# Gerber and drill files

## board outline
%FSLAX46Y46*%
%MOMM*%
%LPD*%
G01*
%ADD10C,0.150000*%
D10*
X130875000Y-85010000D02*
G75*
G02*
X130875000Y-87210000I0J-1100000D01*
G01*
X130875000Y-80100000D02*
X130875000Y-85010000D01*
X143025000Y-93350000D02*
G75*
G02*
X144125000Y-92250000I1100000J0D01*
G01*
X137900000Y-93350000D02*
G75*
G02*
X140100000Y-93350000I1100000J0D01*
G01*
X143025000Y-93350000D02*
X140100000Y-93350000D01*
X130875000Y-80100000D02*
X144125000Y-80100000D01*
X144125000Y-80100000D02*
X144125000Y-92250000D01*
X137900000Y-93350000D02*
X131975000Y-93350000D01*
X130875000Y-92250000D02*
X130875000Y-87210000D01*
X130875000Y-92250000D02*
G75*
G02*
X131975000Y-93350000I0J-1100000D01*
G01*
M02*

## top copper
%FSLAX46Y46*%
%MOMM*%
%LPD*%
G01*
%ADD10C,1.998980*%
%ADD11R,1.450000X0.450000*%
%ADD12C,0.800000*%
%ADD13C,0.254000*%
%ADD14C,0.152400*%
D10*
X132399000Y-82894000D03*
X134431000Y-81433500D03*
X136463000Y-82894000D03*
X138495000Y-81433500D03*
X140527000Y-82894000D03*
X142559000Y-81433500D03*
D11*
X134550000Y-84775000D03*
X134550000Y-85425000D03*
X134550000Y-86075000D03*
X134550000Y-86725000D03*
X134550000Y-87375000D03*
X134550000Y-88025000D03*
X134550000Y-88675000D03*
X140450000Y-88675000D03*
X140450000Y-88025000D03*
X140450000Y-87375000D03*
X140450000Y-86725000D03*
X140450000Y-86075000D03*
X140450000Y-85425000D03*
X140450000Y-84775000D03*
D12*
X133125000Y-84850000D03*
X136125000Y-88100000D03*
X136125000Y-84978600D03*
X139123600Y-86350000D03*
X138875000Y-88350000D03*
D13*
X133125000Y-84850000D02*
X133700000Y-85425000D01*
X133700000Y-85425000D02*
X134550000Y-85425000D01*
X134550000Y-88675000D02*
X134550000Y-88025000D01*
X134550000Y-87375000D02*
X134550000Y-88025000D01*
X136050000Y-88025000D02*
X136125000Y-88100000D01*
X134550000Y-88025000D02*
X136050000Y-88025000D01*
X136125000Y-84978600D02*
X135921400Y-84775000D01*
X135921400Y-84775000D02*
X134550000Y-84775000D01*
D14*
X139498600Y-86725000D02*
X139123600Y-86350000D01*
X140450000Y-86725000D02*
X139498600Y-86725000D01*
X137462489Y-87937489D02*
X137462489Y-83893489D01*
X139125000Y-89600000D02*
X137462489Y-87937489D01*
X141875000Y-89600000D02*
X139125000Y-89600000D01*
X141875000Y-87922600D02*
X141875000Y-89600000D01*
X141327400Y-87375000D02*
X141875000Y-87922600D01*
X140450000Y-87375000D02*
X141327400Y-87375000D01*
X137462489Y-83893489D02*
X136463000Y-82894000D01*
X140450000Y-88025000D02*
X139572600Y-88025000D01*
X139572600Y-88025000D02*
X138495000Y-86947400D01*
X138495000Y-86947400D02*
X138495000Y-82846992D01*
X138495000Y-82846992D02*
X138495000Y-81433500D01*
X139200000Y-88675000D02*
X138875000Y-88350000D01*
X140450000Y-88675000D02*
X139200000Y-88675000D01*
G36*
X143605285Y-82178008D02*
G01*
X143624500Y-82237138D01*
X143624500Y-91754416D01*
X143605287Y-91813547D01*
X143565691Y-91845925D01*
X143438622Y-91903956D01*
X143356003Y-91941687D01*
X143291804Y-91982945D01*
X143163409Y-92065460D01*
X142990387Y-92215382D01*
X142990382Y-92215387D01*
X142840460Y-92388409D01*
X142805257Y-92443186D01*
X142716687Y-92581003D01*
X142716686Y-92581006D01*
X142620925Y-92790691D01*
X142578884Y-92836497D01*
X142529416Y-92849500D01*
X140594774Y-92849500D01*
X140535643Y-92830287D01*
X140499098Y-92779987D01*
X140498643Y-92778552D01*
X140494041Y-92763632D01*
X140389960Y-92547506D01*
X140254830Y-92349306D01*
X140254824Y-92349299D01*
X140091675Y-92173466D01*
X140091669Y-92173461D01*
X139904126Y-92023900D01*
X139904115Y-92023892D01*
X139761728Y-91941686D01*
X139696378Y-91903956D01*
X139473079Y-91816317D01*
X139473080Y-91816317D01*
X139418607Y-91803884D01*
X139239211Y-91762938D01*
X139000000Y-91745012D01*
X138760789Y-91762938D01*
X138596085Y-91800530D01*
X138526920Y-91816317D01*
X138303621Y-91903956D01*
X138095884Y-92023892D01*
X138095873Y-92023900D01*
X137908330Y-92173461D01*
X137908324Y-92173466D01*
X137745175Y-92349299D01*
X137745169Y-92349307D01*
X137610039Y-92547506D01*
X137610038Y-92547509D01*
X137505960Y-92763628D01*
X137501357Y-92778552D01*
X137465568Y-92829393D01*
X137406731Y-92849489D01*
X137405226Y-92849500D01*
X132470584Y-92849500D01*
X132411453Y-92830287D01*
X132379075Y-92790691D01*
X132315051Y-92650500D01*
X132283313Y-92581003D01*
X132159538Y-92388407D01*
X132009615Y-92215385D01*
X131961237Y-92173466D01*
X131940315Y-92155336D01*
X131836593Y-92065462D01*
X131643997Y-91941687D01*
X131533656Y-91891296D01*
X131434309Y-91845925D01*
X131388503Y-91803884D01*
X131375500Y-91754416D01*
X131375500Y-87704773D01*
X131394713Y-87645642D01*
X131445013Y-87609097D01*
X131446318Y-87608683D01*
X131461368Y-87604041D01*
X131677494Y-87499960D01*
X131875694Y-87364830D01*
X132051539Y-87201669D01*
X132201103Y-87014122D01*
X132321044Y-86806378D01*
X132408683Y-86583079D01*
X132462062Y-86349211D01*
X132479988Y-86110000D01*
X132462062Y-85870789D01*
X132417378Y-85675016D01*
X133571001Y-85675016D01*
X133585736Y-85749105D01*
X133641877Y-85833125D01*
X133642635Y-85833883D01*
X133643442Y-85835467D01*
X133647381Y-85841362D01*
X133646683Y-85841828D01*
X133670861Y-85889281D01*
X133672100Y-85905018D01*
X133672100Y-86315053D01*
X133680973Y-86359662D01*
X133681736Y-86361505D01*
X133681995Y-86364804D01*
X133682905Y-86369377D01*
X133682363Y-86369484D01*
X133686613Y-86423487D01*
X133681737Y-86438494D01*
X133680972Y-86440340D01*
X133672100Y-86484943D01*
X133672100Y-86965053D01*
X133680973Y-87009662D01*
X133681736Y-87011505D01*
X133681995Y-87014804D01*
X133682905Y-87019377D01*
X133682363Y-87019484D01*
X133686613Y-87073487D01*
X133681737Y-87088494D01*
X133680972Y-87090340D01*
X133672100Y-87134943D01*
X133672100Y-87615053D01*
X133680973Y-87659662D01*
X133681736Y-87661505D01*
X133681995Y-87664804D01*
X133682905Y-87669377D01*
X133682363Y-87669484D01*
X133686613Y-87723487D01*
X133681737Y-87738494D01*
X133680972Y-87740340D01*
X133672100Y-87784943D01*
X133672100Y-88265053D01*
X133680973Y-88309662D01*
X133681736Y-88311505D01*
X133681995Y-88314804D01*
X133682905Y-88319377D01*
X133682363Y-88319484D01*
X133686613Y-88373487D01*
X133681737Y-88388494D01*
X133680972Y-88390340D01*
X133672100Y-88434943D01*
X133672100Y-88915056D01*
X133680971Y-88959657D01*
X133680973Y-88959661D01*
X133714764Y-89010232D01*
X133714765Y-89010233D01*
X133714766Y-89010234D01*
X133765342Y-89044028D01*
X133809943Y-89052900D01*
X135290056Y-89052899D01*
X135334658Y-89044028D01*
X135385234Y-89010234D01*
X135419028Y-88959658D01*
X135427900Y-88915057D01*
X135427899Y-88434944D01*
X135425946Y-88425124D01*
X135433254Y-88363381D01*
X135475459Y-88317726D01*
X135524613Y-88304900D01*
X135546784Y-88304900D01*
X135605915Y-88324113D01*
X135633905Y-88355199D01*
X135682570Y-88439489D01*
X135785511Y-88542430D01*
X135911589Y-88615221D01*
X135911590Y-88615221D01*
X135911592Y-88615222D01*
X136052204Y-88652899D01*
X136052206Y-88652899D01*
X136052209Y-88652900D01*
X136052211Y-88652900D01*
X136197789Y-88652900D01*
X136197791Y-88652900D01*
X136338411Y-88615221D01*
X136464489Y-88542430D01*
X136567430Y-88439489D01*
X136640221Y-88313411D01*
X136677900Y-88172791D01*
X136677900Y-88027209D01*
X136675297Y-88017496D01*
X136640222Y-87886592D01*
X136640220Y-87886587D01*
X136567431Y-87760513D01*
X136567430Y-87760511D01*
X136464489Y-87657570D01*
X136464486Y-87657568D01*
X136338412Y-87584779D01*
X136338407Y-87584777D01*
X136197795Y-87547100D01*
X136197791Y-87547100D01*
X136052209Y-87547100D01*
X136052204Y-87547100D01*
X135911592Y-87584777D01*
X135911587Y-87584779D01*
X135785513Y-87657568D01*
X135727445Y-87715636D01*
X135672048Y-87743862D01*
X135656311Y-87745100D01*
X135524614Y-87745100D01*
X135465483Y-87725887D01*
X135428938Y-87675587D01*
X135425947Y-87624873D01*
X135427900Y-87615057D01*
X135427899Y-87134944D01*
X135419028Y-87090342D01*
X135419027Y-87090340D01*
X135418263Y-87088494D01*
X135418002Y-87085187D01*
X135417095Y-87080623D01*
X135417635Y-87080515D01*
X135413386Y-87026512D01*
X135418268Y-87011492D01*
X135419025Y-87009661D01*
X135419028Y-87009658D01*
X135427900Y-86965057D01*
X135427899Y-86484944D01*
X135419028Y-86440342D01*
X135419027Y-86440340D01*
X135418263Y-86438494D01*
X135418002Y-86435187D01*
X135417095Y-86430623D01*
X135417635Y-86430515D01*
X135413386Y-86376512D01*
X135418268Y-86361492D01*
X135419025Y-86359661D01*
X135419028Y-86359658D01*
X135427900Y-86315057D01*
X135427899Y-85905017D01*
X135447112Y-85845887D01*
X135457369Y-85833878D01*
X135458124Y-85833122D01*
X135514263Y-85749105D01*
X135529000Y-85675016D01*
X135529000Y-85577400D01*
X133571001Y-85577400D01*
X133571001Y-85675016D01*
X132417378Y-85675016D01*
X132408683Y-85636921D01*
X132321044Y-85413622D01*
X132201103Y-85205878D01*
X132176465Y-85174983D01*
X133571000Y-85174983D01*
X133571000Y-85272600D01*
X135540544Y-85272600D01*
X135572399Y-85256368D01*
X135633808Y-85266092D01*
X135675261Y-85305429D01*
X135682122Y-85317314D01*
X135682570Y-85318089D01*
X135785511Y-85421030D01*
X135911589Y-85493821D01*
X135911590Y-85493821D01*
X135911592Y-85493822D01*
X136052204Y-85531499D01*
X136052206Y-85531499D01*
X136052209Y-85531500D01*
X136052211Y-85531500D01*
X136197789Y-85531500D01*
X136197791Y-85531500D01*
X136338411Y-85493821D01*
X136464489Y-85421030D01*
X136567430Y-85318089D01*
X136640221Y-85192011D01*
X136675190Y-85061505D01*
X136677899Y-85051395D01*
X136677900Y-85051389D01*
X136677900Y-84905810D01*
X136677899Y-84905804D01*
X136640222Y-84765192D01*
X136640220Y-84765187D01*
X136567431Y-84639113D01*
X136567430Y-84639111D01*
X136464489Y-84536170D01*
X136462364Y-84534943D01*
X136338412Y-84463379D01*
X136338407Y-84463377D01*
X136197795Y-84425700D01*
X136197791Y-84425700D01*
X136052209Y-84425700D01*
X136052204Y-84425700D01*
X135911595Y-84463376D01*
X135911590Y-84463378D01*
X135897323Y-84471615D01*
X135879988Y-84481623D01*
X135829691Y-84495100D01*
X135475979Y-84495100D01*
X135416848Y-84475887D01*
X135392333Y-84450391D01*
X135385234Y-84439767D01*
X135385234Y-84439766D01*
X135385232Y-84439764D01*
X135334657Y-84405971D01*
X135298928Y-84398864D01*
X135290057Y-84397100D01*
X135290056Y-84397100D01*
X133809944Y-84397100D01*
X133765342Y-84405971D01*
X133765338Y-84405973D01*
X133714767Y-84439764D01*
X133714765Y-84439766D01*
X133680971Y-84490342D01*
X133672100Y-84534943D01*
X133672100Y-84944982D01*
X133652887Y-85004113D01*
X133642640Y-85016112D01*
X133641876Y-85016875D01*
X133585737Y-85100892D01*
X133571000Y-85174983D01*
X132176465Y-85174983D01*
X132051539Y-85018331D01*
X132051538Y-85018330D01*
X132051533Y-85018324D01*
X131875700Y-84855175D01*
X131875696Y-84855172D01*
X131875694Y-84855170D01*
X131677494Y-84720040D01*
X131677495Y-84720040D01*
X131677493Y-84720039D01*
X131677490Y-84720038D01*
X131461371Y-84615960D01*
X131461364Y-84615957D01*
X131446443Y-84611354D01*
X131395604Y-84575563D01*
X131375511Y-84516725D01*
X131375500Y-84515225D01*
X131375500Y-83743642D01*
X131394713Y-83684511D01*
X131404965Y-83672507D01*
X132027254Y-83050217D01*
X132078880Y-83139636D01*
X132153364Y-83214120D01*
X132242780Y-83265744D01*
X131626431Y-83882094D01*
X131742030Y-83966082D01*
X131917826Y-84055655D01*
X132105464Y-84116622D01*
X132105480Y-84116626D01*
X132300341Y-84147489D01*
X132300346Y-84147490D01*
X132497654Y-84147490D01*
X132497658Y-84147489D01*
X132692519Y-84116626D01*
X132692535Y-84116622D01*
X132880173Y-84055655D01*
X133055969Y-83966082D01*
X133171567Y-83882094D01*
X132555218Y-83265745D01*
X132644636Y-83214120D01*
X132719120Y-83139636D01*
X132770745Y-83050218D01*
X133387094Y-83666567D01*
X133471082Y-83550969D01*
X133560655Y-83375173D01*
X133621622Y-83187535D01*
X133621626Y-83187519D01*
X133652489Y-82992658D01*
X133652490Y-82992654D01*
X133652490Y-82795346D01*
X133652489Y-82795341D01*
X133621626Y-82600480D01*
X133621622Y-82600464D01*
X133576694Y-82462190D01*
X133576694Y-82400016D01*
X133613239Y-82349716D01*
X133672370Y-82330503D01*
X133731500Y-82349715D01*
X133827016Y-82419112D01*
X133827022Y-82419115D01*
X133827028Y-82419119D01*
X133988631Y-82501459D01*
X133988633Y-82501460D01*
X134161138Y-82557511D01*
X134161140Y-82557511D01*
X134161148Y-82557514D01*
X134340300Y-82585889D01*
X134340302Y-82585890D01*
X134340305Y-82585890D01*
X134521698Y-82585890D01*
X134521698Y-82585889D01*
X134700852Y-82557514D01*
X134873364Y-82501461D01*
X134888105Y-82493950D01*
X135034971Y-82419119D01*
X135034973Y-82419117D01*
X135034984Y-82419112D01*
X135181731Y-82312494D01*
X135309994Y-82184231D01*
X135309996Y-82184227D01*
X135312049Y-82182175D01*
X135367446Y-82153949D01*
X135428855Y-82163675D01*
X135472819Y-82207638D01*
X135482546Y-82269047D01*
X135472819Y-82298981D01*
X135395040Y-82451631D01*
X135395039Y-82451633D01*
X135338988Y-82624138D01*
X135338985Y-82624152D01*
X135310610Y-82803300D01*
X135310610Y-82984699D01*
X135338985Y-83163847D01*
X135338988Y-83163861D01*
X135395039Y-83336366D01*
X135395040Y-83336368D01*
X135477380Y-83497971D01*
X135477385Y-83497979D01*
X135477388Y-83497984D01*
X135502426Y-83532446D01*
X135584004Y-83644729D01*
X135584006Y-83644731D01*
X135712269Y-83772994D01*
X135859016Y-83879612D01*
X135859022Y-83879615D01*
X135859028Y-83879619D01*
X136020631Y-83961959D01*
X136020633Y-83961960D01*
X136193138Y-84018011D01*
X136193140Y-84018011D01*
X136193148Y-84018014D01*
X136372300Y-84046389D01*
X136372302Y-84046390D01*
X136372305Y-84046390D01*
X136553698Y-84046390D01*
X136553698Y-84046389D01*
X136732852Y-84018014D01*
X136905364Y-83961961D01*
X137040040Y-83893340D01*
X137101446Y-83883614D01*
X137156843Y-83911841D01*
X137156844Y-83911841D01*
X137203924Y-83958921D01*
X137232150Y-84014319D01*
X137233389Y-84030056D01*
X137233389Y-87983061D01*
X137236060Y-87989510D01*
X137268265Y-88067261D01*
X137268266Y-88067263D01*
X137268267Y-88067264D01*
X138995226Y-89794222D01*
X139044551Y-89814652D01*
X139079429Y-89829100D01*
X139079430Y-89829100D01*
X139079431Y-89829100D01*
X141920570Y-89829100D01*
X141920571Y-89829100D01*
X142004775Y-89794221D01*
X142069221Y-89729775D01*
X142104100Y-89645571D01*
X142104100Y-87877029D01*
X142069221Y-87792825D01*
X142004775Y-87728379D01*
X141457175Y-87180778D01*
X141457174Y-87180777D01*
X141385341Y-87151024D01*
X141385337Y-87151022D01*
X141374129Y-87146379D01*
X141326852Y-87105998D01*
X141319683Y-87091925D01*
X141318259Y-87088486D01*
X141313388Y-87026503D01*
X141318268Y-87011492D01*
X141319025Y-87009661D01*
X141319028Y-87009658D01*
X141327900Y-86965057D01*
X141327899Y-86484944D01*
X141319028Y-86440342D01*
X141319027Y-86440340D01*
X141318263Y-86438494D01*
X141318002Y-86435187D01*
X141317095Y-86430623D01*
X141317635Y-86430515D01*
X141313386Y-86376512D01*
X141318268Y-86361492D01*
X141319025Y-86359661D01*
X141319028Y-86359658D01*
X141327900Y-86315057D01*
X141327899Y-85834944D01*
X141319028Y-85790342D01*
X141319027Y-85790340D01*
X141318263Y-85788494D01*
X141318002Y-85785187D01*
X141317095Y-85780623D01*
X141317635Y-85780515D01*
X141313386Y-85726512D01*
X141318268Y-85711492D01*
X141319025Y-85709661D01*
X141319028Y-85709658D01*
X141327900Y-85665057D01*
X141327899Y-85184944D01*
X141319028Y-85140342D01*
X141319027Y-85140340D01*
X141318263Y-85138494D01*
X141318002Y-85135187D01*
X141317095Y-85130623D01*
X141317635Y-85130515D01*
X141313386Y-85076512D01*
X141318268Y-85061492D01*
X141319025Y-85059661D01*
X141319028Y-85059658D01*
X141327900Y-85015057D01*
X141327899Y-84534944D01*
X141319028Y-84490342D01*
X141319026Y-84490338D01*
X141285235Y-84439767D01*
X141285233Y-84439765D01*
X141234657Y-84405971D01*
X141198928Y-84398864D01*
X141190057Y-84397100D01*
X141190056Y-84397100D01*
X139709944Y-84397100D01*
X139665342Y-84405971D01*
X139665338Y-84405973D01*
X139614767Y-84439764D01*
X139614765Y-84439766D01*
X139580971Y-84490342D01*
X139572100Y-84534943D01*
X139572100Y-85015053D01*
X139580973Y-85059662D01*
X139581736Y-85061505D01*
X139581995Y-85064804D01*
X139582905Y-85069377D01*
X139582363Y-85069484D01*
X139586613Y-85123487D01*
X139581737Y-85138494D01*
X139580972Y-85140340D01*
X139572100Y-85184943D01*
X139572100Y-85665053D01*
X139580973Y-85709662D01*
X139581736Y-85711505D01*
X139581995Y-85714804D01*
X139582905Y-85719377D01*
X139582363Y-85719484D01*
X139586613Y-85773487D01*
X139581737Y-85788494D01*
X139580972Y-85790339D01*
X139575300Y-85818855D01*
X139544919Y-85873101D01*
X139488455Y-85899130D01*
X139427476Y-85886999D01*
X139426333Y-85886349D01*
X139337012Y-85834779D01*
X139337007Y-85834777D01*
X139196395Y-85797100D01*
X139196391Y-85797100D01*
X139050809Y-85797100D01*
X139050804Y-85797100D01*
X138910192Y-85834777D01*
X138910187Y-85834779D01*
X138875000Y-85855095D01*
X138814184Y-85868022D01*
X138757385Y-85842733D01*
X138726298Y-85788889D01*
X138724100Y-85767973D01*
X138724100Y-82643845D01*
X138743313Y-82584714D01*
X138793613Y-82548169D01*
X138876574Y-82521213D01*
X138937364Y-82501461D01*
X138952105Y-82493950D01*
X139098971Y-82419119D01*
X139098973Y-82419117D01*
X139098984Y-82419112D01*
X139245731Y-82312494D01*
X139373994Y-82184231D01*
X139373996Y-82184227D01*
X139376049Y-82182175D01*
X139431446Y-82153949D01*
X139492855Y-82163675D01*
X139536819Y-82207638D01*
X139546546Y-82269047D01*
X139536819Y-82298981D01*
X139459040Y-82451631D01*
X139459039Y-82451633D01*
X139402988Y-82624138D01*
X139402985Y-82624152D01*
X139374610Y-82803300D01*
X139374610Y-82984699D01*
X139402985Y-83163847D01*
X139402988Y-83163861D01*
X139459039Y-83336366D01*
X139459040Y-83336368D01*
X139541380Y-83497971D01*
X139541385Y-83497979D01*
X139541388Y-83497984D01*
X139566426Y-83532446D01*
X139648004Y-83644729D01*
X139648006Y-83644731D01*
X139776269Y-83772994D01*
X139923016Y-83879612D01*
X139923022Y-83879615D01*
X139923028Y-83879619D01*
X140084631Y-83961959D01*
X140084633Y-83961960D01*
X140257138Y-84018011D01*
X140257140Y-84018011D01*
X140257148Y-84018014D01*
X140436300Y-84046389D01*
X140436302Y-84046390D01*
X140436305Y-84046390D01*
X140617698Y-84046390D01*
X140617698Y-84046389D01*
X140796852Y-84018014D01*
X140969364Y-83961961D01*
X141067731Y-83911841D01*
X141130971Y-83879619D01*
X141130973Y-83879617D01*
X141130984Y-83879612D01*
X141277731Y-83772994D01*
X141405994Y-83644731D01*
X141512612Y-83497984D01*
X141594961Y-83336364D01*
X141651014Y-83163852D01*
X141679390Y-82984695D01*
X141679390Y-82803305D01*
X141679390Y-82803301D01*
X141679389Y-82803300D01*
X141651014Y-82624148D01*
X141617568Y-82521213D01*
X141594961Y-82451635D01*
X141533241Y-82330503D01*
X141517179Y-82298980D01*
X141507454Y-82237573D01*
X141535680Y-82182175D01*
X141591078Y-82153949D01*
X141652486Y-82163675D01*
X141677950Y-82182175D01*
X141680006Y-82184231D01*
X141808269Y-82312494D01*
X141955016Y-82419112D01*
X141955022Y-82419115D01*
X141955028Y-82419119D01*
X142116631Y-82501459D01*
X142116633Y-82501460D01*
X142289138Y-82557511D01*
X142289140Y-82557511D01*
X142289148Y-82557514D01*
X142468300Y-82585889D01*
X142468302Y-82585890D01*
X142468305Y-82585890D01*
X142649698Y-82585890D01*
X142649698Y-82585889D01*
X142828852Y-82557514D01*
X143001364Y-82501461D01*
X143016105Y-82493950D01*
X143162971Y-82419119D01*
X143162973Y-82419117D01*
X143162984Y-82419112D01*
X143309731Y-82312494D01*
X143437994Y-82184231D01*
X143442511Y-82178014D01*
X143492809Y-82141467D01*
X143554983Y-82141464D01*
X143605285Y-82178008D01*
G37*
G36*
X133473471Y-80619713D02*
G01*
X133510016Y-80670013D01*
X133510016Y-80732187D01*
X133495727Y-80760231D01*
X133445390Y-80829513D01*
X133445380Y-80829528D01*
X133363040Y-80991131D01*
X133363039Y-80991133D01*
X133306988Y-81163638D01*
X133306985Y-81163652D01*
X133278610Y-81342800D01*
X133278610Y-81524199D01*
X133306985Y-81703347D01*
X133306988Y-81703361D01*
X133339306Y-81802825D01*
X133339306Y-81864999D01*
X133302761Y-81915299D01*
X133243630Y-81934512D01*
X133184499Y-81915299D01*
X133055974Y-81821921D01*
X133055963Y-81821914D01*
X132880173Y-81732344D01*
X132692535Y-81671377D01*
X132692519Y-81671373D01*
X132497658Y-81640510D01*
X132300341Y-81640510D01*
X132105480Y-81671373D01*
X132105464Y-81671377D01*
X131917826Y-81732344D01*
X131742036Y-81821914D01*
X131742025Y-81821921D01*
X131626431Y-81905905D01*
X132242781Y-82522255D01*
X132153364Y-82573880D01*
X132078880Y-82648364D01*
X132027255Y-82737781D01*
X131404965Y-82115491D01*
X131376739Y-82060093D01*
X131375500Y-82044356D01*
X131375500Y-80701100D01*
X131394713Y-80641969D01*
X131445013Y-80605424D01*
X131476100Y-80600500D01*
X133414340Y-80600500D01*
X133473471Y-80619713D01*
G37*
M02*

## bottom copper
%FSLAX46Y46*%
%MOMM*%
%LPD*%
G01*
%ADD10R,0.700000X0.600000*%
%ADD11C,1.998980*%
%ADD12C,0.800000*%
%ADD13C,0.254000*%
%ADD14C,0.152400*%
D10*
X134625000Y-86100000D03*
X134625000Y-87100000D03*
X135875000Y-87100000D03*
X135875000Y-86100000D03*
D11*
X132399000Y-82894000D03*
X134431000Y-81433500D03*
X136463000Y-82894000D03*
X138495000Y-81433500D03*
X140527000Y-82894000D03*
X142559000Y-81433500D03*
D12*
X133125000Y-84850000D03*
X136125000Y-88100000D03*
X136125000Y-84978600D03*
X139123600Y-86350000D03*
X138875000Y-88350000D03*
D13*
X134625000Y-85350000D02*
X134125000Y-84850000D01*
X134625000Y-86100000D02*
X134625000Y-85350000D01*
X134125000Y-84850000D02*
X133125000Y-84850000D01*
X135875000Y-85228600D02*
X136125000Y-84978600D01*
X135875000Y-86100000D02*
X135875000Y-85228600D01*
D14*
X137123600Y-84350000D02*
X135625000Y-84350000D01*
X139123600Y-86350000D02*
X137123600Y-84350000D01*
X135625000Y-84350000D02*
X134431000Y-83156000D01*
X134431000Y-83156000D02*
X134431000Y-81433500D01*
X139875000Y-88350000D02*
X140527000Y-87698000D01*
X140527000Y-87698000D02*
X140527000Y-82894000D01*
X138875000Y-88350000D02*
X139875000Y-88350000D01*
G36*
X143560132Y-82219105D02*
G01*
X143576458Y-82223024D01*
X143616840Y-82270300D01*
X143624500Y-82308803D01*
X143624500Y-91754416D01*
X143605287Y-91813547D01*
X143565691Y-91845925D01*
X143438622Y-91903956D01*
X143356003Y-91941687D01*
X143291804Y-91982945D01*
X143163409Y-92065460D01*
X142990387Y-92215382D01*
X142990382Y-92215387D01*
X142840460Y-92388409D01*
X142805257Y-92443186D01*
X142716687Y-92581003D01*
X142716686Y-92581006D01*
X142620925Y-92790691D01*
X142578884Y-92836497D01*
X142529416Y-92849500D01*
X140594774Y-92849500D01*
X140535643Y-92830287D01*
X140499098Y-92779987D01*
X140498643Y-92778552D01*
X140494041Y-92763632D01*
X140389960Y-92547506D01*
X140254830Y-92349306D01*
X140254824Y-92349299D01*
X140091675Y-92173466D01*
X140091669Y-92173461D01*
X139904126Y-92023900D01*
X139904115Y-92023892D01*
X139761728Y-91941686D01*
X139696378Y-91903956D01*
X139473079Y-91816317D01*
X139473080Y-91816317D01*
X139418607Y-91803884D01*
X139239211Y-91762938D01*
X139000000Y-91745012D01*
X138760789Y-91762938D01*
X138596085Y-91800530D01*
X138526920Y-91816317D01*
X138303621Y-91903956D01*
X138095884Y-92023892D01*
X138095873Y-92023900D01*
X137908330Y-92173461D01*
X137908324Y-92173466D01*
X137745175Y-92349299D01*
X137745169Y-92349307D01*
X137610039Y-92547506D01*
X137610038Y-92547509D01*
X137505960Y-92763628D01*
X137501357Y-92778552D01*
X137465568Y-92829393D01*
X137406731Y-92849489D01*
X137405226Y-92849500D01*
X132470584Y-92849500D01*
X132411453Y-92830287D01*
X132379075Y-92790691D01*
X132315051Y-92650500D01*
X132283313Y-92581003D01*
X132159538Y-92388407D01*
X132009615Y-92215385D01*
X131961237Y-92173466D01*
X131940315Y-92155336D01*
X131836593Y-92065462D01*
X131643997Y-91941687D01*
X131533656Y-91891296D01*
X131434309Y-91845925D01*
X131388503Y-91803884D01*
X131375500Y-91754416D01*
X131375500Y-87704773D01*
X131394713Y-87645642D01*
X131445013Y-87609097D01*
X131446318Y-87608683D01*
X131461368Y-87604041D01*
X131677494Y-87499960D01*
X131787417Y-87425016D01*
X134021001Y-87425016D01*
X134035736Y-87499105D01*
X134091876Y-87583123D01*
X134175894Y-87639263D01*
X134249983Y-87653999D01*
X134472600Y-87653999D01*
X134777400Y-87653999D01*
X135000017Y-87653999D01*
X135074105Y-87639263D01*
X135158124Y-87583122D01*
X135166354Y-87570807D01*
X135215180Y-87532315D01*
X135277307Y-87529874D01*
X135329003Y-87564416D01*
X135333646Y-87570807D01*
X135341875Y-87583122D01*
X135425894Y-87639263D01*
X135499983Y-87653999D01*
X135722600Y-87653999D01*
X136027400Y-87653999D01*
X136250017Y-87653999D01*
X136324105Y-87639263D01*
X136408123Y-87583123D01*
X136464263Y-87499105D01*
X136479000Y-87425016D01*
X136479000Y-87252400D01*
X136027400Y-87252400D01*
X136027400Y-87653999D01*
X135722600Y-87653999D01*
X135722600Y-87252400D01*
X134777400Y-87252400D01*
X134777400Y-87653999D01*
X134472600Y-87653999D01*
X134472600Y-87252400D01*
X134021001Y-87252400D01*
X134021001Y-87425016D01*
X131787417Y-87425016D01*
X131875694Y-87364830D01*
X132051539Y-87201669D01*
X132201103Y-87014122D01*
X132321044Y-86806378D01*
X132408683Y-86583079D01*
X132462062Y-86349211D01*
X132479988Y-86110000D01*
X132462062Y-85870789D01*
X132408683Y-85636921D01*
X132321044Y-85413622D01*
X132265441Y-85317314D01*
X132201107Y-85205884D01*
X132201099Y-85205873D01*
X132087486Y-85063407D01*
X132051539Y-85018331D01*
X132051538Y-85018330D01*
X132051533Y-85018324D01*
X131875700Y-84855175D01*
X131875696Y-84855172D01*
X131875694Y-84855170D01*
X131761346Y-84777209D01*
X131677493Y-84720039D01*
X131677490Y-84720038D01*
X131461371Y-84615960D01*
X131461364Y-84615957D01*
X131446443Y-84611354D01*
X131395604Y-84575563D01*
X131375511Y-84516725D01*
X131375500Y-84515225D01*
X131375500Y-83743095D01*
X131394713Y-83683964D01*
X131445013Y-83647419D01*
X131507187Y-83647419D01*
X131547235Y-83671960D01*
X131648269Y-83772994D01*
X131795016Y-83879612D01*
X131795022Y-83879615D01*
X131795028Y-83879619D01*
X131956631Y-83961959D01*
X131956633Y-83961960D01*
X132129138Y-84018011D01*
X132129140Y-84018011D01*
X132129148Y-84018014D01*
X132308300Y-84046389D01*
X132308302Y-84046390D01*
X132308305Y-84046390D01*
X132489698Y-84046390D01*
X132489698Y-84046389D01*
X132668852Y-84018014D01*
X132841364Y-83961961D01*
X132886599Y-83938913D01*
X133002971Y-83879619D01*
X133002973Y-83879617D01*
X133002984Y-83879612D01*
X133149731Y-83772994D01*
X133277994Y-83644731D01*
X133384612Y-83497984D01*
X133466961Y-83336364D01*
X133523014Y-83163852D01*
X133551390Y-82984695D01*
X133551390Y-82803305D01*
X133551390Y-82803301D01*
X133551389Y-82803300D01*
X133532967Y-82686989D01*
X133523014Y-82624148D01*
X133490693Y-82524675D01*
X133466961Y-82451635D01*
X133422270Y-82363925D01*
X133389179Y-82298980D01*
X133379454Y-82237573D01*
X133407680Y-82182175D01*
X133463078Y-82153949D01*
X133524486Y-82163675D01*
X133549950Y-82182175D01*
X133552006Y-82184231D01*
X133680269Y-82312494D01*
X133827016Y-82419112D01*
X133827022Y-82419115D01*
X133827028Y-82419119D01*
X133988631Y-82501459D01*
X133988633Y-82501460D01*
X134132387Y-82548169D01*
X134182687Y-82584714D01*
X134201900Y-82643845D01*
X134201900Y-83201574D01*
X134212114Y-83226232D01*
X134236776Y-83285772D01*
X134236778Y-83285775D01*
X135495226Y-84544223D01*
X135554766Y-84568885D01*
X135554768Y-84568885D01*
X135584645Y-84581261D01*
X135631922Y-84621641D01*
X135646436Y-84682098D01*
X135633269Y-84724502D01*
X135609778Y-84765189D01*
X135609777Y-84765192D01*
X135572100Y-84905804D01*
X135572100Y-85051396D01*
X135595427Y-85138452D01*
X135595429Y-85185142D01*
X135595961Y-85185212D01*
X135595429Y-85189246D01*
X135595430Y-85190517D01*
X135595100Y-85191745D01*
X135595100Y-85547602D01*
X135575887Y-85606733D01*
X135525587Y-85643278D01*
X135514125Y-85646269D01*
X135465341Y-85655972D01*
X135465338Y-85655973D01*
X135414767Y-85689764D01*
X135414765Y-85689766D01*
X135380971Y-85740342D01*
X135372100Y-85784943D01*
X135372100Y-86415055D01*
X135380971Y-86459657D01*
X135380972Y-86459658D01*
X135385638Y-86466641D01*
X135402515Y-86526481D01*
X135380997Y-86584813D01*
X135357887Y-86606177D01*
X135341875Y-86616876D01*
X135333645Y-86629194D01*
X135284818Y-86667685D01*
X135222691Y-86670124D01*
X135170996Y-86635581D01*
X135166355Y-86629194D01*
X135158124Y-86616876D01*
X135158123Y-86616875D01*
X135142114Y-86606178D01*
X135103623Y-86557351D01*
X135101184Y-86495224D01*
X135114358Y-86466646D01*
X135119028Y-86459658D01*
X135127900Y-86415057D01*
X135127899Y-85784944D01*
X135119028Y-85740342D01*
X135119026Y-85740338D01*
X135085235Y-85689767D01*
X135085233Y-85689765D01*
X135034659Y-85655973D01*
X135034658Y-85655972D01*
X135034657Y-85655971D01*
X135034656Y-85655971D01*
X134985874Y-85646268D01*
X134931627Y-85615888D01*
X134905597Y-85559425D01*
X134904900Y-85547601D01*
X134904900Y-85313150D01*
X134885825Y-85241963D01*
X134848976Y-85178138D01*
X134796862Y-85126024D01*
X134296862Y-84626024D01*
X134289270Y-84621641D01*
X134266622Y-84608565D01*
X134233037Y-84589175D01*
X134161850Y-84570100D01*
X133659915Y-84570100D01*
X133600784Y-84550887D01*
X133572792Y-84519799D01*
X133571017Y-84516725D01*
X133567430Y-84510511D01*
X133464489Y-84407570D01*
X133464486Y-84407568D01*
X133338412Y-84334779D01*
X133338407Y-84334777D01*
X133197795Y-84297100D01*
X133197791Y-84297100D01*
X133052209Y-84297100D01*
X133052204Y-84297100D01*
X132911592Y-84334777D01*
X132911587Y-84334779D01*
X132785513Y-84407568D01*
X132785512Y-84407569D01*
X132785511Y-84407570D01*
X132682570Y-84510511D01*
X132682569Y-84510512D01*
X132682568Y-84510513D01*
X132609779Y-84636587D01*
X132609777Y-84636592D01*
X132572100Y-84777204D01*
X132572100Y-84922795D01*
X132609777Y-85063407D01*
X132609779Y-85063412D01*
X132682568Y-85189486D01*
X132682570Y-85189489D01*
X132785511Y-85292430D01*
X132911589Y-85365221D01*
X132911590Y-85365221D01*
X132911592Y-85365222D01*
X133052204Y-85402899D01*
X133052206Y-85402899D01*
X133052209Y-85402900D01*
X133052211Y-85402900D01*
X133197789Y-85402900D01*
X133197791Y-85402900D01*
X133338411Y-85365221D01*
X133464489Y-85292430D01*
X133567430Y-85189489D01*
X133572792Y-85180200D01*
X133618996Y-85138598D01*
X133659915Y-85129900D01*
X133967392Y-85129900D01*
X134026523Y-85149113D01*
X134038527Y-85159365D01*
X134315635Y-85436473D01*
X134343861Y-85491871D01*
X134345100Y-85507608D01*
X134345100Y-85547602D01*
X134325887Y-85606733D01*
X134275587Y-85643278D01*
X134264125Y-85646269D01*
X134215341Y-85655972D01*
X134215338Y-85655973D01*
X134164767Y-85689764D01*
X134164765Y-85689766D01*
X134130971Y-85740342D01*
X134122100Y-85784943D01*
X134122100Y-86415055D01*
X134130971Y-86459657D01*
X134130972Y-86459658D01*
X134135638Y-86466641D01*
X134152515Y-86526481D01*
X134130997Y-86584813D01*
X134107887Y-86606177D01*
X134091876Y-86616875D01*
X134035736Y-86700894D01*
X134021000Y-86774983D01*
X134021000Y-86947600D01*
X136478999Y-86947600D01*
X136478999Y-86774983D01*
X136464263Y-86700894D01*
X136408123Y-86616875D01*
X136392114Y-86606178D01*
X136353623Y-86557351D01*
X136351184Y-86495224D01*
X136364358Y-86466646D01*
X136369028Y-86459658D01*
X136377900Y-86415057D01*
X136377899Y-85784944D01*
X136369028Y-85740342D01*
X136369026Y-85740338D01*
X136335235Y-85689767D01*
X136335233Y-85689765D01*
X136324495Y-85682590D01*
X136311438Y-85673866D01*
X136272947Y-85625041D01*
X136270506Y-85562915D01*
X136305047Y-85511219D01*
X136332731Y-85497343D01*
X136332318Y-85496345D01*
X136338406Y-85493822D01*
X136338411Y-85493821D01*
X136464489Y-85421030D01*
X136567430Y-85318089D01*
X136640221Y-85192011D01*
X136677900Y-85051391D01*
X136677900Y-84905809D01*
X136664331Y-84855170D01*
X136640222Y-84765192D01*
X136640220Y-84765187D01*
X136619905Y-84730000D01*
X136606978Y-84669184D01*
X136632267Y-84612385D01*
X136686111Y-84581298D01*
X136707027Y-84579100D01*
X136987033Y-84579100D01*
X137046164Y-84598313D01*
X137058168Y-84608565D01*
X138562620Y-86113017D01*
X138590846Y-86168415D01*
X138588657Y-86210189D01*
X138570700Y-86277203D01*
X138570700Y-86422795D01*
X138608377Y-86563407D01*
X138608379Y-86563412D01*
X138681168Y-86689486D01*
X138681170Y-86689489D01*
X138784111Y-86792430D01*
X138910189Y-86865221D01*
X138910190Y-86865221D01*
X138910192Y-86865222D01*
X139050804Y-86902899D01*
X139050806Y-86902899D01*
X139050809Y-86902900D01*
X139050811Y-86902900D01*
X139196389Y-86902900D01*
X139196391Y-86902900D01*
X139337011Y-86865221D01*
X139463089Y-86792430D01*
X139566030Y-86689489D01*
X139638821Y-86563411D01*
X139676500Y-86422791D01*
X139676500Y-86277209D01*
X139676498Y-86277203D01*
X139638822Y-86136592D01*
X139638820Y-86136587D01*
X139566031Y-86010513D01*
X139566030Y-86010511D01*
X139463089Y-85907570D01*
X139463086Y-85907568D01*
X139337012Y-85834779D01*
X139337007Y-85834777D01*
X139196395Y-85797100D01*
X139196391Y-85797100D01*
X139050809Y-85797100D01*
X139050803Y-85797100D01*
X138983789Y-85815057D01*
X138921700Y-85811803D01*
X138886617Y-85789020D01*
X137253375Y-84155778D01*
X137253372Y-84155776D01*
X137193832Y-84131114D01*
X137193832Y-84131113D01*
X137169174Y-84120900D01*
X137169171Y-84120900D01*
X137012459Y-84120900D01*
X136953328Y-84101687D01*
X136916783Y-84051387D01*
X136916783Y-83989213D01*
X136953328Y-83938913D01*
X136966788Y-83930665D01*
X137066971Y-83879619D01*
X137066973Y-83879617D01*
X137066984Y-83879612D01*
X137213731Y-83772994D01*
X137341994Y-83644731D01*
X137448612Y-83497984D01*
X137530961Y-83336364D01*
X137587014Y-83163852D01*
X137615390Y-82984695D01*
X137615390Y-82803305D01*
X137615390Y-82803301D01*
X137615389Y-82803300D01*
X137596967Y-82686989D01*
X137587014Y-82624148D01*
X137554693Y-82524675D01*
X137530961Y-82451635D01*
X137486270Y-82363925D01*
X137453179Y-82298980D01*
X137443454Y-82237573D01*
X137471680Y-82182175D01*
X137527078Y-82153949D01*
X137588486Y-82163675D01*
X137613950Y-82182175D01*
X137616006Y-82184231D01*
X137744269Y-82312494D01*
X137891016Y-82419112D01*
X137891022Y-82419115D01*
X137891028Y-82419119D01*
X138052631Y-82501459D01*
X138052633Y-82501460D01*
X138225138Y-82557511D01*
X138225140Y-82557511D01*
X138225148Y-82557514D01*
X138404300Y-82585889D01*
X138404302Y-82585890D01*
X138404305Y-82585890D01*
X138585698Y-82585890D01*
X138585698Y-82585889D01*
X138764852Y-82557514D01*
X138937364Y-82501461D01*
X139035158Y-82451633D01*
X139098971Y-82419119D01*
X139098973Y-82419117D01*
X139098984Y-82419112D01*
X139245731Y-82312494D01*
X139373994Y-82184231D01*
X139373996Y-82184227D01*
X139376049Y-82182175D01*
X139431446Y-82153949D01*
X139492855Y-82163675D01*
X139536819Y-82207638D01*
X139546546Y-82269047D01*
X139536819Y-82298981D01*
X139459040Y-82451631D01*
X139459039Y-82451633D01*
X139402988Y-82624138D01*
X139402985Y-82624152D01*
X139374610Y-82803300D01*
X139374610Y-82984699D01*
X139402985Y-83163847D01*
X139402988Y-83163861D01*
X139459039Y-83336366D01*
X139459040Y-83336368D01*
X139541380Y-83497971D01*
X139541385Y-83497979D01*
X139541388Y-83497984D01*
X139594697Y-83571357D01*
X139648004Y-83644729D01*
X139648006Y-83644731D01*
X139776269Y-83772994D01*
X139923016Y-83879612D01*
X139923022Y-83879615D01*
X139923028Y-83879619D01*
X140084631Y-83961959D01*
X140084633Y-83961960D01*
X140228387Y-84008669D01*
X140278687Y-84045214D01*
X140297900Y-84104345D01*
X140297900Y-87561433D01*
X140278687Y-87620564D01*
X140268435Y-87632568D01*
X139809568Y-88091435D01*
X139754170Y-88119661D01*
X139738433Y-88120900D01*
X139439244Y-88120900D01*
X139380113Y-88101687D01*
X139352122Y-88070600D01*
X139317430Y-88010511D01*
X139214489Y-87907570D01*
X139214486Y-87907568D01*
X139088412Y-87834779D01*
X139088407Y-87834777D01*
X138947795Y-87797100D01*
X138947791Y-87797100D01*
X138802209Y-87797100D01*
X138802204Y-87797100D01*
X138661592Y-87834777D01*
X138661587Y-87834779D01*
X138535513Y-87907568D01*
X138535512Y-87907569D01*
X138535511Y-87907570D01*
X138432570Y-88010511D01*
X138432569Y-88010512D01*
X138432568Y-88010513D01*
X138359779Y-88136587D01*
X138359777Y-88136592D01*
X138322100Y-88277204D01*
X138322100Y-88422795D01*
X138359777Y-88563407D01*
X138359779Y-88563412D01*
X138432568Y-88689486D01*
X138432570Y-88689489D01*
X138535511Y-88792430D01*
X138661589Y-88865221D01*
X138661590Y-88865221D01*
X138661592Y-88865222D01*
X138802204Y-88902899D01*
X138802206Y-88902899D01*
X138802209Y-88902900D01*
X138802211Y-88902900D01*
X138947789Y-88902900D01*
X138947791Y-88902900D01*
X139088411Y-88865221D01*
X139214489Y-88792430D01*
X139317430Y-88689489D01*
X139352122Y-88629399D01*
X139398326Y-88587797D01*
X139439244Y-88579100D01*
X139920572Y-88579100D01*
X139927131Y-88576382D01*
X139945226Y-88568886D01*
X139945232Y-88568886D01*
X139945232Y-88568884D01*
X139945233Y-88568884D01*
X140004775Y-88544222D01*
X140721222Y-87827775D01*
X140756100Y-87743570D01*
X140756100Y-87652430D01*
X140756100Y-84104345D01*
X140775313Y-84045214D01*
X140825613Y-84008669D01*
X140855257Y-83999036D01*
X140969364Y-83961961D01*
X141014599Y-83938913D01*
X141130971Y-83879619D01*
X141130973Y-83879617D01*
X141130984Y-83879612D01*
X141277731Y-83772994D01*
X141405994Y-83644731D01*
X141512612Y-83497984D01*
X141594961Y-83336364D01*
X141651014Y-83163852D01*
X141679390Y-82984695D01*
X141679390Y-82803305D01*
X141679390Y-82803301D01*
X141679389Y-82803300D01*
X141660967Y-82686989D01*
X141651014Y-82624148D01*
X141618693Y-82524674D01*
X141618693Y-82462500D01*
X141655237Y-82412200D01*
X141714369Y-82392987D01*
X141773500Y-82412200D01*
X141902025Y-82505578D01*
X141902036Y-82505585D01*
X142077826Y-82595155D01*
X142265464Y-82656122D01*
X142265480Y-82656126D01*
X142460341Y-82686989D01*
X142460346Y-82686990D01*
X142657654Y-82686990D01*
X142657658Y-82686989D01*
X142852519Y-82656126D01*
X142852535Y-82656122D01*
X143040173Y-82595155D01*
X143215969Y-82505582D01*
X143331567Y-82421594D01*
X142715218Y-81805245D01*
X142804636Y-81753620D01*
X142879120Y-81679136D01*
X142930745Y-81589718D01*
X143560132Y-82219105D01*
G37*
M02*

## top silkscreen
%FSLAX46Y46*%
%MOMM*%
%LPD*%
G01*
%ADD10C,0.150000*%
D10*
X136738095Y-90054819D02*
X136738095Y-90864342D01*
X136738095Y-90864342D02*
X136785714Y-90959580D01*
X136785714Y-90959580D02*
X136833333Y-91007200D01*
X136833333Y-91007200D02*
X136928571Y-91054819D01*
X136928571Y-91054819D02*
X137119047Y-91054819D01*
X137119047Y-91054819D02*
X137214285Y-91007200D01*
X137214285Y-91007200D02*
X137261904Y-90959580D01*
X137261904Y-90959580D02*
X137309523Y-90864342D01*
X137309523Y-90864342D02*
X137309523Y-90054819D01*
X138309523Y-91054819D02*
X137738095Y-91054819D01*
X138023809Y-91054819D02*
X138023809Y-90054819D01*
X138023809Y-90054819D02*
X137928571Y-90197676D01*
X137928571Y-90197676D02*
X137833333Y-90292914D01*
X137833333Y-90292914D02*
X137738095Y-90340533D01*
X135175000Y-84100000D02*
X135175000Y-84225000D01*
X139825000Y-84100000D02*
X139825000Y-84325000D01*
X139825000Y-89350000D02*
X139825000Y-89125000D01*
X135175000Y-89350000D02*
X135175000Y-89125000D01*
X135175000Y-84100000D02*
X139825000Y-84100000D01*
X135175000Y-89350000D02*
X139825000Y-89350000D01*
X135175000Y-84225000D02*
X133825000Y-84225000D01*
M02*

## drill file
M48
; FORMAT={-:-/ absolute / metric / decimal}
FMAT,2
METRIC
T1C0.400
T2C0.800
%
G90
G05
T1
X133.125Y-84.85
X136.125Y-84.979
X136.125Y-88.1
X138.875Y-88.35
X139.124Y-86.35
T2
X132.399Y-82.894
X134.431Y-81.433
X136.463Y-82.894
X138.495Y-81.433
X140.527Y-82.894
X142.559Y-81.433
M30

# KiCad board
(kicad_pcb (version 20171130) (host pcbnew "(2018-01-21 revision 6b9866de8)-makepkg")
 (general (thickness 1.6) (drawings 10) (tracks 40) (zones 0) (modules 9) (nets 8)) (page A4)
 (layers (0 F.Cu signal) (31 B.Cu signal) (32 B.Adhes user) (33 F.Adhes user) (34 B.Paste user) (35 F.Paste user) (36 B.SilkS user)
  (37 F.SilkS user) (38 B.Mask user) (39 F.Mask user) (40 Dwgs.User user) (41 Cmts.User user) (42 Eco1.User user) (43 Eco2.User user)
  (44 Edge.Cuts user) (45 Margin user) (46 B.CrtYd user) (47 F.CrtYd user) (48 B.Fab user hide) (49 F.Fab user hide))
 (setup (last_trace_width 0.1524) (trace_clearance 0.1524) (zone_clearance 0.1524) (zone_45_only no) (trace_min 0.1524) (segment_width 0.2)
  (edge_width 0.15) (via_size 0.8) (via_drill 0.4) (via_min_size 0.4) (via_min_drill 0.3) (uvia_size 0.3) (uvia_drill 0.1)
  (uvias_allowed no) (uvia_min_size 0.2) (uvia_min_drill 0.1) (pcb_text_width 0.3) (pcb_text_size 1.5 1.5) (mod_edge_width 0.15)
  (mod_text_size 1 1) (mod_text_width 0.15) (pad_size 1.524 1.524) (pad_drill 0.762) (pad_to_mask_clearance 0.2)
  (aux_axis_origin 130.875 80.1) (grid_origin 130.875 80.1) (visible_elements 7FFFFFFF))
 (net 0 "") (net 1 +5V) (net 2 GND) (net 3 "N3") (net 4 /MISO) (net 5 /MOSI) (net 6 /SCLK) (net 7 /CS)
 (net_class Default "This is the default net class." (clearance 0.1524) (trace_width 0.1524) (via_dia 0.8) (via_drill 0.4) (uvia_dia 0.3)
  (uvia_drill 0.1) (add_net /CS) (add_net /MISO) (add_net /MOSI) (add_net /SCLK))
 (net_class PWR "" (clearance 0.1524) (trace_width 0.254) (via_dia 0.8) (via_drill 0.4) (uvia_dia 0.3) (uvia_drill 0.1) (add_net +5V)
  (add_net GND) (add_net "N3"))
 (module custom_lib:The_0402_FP (layer B.Cu) (at 134.625 86.6 90)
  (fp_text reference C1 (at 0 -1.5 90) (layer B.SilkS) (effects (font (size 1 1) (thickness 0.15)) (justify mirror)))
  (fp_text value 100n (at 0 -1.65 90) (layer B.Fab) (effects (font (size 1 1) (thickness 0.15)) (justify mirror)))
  (pad 2 smd rect (at 0.5 0 90) (size 0.6 0.7) (layers B.Cu B.Paste B.Mask) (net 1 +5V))
  (pad 1 smd rect (at -0.5 0 90) (size 0.6 0.7) (layers B.Cu B.Paste B.Mask) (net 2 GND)))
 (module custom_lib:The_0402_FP (layer B.Cu) (at 135.875 86.6 90)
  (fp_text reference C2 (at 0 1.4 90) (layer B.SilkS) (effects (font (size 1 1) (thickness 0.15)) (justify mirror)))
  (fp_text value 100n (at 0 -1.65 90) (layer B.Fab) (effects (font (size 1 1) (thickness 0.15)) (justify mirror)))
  (pad 1 smd rect (at -0.5 0 90) (size 0.6 0.7) (layers B.Cu B.Paste B.Mask) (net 2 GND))
  (pad 2 smd rect (at 0.5 0 90) (size 0.6 0.7) (layers B.Cu B.Paste B.Mask) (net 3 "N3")))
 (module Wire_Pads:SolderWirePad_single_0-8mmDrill (layer F.Cu) (at 132.399 82.894)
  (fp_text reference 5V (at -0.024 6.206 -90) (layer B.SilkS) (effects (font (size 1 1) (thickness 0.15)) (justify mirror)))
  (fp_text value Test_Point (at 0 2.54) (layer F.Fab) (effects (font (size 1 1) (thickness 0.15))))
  (pad 1 thru_hole circle (at 0 0) (size 1.99898 1.99898) (drill 0.8001) (layers *.Cu *.Mask) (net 1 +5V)))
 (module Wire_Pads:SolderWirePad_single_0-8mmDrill (layer F.Cu) (at 134.431 81.4335)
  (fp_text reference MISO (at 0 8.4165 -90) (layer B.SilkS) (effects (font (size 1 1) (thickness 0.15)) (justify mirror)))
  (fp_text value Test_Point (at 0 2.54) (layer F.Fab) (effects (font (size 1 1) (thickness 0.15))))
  (pad 1 thru_hole circle (at 0 0) (size 1.99898 1.99898) (drill 0.8001) (layers *.Cu *.Mask) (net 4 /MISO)))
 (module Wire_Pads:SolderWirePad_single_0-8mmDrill (layer F.Cu) (at 136.463 82.894)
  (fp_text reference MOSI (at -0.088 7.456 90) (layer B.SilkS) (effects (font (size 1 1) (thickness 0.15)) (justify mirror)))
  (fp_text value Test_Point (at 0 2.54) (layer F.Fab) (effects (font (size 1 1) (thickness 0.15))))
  (pad 1 thru_hole circle (at 0 0) (size 1.99898 1.99898) (drill 0.8001) (layers *.Cu *.Mask) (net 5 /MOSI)))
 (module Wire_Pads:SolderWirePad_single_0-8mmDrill (layer F.Cu) (at 138.495 81.4335)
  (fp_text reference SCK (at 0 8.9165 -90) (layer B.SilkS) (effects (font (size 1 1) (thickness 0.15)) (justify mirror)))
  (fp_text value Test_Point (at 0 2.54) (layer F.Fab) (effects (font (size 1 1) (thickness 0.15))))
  (pad 1 thru_hole circle (at 0 0) (size 1.99898 1.99898) (drill 0.8001) (layers *.Cu *.Mask) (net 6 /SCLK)))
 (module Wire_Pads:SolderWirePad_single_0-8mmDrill (layer F.Cu) (at 140.527 82.894)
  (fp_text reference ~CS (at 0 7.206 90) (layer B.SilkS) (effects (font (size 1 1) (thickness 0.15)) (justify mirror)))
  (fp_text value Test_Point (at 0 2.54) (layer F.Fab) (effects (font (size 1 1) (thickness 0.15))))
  (pad 1 thru_hole circle (at 0 0) (size 1.99898 1.99898) (drill 0.8001) (layers *.Cu *.Mask) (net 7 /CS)))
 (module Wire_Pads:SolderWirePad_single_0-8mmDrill (layer F.Cu) (at 142.559 81.4335)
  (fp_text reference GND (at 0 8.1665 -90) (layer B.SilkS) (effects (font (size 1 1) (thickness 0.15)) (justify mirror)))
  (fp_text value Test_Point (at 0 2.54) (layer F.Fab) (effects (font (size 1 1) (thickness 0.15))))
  (pad 1 thru_hole circle (at 0 0) (size 1.99898 1.99898) (drill 0.8001) (layers *.Cu *.Mask) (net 2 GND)))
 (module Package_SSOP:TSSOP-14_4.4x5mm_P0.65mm (layer F.Cu) (at 137.5 86.725)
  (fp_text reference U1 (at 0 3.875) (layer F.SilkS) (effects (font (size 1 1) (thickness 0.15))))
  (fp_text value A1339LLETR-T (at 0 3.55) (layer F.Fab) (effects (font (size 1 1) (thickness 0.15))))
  (fp_line (start -2.325 -2.625) (end -2.325 -2.5) (layer F.SilkS) (width 0.15))
  (fp_line (start 2.325 -2.625) (end 2.325 -2.4) (layer F.SilkS) (width 0.15))
  (fp_line (start 2.325 2.625) (end 2.325 2.4) (layer F.SilkS) (width 0.15))
  (fp_line (start -2.325 2.625) (end -2.325 2.4) (layer F.SilkS) (width 0.15))
  (fp_line (start -2.325 -2.625) (end 2.325 -2.625) (layer F.SilkS) (width 0.15))
  (fp_line (start -2.325 2.625) (end 2.325 2.625) (layer F.SilkS) (width 0.15))
  (fp_line (start -2.325 -2.5) (end -3.675 -2.5) (layer F.SilkS) (width 0.15))
  (pad 1 smd rect (at -2.95 -1.95) (size 1.45 0.45) (layers F.Cu F.Paste F.Mask) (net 3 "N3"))
  (pad 2 smd rect (at -2.95 -1.3) (size 1.45 0.45) (layers F.Cu F.Paste F.Mask) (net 1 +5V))
  (pad 3 smd rect (at -2.95 -0.65) (size 1.45 0.45) (layers F.Cu F.Paste F.Mask))
  (pad 4 smd rect (at -2.95 0) (size 1.45 0.45) (layers F.Cu F.Paste F.Mask))
  (pad 5 smd rect (at -2.95 0.65) (size 1.45 0.45) (layers F.Cu F.Paste F.Mask) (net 2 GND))
  (pad 6 smd rect (at -2.95 1.3) (size 1.45 0.45) (layers F.Cu F.Paste F.Mask) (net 2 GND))
  (pad 7 smd rect (at -2.95 1.95) (size 1.45 0.45) (layers F.Cu F.Paste F.Mask) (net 2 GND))
  (pad 8 smd rect (at 2.95 1.95) (size 1.45 0.45) (layers F.Cu F.Paste F.Mask) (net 7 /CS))
  (pad 9 smd rect (at 2.95 1.3) (size 1.45 0.45) (layers F.Cu F.Paste F.Mask) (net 6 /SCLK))
  (pad 10 smd rect (at 2.95 0.65) (size 1.45 0.45) (layers F.Cu F.Paste F.Mask) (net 5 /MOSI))
  (pad 11 smd rect (at 2.95 0) (size 1.45 0.45) (layers F.Cu F.Paste F.Mask) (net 4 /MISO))
  (pad 12 smd rect (at 2.95 -0.65) (size 1.45 0.45) (layers F.Cu F.Paste F.Mask))
  (pad 13 smd rect (at 2.95 -1.3) (size 1.45 0.45) (layers F.Cu F.Paste F.Mask))
  (pad 14 smd rect (at 2.95 -1.95) (size 1.45 0.45) (layers F.Cu F.Paste F.Mask)))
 (gr_arc (start 130.875 86.11) (end 130.875 85.01) (angle 180) (layer Edge.Cuts) (width 0.15))
 (gr_line (start 130.875 80.1) (end 130.875 85.01) (angle 90) (layer Edge.Cuts) (width 0.15))
 (gr_arc (start 144.125 93.35) (end 143.025 93.35) (angle 90) (layer Edge.Cuts) (width 0.15))
 (gr_arc (start 139 93.35) (end 137.9 93.35) (angle 180) (layer Edge.Cuts) (width 0.15))
 (gr_line (start 143.025 93.35) (end 140.1 93.35) (angle 90) (layer Edge.Cuts) (width 0.15))
 (gr_line (start 130.875 80.1) (end 144.125 80.1) (angle 90) (layer Edge.Cuts) (width 0.15))
 (gr_line (start 144.125 80.1) (end 144.125 92.25) (angle 90) (layer Edge.Cuts) (width 0.15))
 (gr_line (start 137.9 93.35) (end 131.975 93.35) (angle 90) (layer Edge.Cuts) (width 0.15))
 (gr_line (start 130.875 92.25) (end 130.875 87.21) (angle 90) (layer Edge.Cuts) (width 0.15))
 (gr_arc (start 130.875 93.35) (end 130.875 92.25) (angle 90) (layer Edge.Cuts) (width 0.15))
 (segment (start 134.625 85.35) (end 134.125 84.85) (width 0.254) (layer B.Cu) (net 1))
 (segment (start 134.625 86.1) (end 134.625 85.35) (width 0.254) (layer B.Cu) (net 1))
 (segment (start 134.125 84.85) (end 133.125 84.85) (width 0.254) (layer B.Cu) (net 1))
 (segment (start 133.125 84.85) (end 133.7 85.425) (width 0.254) (layer F.Cu) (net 1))
 (segment (start 133.7 85.425) (end 134.55 85.425) (width 0.254) (layer F.Cu) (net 1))
 (via (at 133.125 84.85) (size 0.8) (drill 0.4) (layers F.Cu B.Cu) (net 1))
 (segment (start 134.55 88.675) (end 134.55 88.025) (width 0.254) (layer F.Cu) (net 2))
 (segment (start 134.55 87.375) (end 134.55 88.025) (width 0.254) (layer F.Cu) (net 2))
 (segment (start 136.05 88.025) (end 136.125 88.1) (width 0.254) (layer F.Cu) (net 2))
 (segment (start 134.55 88.025) (end 136.05 88.025) (width 0.254) (layer F.Cu) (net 2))
 (via (at 136.125 88.1) (size 0.8) (drill 0.4) (layers F.Cu B.Cu) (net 2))
 (segment (start 136.125 84.9786) (end 135.9214 84.775) (width 0.254) (layer F.Cu) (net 3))
 (segment (start 135.9214 84.775) (end 134.55 84.775) (width 0.254) (layer F.Cu) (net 3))
 (segment (start 135.875 85.2286) (end 136.125 84.9786) (width 0.254) (layer B.Cu) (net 3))
 (segment (start 135.875 86.1) (end 135.875 85.2286) (width 0.254) (layer B.Cu) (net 3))
 (via (at 136.125 84.9786) (size 0.8) (drill 0.4) (layers F.Cu B.Cu) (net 3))
 (segment (start 137.1236 84.35) (end 135.625 84.35) (width 0.1524) (layer B.Cu) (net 4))
 (segment (start 139.1236 86.35) (end 137.1236 84.35) (width 0.1524) (layer B.Cu) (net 4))
 (segment (start 135.625 84.35) (end 134.431 83.156) (width 0.1524) (layer B.Cu) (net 4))
 (segment (start 134.431 83.156) (end 134.431 81.4335) (width 0.1524) (layer B.Cu) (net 4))
 (segment (start 139.4986 86.725) (end 139.1236 86.35) (width 0.1524) (layer F.Cu) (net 4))
 (segment (start 140.45 86.725) (end 139.4986 86.725) (width 0.1524) (layer F.Cu) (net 4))
 (via (at 139.1236 86.35) (size 0.8) (drill 0.4) (layers F.Cu B.Cu) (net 4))
 (segment (start 137.462489 87.937489) (end 137.462489 83.893489) (width 0.1524) (layer F.Cu) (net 5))
 (segment (start 139.125 89.6) (end 137.462489 87.937489) (width 0.1524) (layer F.Cu) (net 5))
 (segment (start 141.875 89.6) (end 139.125 89.6) (width 0.1524) (layer F.Cu) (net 5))
 (segment (start 141.875 87.9226) (end 141.875 89.6) (width 0.1524) (layer F.Cu) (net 5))
 (segment (start 141.3274 87.375) (end 141.875 87.9226) (width 0.1524) (layer F.Cu) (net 5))
 (segment (start 140.45 87.375) (end 141.3274 87.375) (width 0.1524) (layer F.Cu) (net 5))
 (segment (start 137.462489 83.893489) (end 136.463 82.894) (width 0.1524) (layer F.Cu) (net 5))
 (segment (start 140.45 88.025) (end 139.5726 88.025) (width 0.1524) (layer F.Cu) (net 6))
 (segment (start 139.5726 88.025) (end 138.495 86.9474) (width 0.1524) (layer F.Cu) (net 6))
 (segment (start 138.495 86.9474) (end 138.495 82.846992) (width 0.1524) (layer F.Cu) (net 6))
 (segment (start 138.495 82.846992) (end 138.495 81.4335) (width 0.1524) (layer F.Cu) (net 6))
 (segment (start 139.875 88.35) (end 140.527 87.698) (width 0.1524) (layer B.Cu) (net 7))
 (segment (start 140.527 87.698) (end 140.527 82.894) (width 0.1524) (layer B.Cu) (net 7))
 (segment (start 138.875 88.35) (end 139.875 88.35) (width 0.1524) (layer B.Cu) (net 7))
 (segment (start 139.2 88.675) (end 138.875 88.35) (width 0.1524) (layer F.Cu) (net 7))
 (segment (start 140.45 88.675) (end 139.2 88.675) (width 0.1524) (layer F.Cu) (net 7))
 (via (at 138.875 88.35) (size 0.8) (drill 0.4) (layers F.Cu B.Cu) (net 7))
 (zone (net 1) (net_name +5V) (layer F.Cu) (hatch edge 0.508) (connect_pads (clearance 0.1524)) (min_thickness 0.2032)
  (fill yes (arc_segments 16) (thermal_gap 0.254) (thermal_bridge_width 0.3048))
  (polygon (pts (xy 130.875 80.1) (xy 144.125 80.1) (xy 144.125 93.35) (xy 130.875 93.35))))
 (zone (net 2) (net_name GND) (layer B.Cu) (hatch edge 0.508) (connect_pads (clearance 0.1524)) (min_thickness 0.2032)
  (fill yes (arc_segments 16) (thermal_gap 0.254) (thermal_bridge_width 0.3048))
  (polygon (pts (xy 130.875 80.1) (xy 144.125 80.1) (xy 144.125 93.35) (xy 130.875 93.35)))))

